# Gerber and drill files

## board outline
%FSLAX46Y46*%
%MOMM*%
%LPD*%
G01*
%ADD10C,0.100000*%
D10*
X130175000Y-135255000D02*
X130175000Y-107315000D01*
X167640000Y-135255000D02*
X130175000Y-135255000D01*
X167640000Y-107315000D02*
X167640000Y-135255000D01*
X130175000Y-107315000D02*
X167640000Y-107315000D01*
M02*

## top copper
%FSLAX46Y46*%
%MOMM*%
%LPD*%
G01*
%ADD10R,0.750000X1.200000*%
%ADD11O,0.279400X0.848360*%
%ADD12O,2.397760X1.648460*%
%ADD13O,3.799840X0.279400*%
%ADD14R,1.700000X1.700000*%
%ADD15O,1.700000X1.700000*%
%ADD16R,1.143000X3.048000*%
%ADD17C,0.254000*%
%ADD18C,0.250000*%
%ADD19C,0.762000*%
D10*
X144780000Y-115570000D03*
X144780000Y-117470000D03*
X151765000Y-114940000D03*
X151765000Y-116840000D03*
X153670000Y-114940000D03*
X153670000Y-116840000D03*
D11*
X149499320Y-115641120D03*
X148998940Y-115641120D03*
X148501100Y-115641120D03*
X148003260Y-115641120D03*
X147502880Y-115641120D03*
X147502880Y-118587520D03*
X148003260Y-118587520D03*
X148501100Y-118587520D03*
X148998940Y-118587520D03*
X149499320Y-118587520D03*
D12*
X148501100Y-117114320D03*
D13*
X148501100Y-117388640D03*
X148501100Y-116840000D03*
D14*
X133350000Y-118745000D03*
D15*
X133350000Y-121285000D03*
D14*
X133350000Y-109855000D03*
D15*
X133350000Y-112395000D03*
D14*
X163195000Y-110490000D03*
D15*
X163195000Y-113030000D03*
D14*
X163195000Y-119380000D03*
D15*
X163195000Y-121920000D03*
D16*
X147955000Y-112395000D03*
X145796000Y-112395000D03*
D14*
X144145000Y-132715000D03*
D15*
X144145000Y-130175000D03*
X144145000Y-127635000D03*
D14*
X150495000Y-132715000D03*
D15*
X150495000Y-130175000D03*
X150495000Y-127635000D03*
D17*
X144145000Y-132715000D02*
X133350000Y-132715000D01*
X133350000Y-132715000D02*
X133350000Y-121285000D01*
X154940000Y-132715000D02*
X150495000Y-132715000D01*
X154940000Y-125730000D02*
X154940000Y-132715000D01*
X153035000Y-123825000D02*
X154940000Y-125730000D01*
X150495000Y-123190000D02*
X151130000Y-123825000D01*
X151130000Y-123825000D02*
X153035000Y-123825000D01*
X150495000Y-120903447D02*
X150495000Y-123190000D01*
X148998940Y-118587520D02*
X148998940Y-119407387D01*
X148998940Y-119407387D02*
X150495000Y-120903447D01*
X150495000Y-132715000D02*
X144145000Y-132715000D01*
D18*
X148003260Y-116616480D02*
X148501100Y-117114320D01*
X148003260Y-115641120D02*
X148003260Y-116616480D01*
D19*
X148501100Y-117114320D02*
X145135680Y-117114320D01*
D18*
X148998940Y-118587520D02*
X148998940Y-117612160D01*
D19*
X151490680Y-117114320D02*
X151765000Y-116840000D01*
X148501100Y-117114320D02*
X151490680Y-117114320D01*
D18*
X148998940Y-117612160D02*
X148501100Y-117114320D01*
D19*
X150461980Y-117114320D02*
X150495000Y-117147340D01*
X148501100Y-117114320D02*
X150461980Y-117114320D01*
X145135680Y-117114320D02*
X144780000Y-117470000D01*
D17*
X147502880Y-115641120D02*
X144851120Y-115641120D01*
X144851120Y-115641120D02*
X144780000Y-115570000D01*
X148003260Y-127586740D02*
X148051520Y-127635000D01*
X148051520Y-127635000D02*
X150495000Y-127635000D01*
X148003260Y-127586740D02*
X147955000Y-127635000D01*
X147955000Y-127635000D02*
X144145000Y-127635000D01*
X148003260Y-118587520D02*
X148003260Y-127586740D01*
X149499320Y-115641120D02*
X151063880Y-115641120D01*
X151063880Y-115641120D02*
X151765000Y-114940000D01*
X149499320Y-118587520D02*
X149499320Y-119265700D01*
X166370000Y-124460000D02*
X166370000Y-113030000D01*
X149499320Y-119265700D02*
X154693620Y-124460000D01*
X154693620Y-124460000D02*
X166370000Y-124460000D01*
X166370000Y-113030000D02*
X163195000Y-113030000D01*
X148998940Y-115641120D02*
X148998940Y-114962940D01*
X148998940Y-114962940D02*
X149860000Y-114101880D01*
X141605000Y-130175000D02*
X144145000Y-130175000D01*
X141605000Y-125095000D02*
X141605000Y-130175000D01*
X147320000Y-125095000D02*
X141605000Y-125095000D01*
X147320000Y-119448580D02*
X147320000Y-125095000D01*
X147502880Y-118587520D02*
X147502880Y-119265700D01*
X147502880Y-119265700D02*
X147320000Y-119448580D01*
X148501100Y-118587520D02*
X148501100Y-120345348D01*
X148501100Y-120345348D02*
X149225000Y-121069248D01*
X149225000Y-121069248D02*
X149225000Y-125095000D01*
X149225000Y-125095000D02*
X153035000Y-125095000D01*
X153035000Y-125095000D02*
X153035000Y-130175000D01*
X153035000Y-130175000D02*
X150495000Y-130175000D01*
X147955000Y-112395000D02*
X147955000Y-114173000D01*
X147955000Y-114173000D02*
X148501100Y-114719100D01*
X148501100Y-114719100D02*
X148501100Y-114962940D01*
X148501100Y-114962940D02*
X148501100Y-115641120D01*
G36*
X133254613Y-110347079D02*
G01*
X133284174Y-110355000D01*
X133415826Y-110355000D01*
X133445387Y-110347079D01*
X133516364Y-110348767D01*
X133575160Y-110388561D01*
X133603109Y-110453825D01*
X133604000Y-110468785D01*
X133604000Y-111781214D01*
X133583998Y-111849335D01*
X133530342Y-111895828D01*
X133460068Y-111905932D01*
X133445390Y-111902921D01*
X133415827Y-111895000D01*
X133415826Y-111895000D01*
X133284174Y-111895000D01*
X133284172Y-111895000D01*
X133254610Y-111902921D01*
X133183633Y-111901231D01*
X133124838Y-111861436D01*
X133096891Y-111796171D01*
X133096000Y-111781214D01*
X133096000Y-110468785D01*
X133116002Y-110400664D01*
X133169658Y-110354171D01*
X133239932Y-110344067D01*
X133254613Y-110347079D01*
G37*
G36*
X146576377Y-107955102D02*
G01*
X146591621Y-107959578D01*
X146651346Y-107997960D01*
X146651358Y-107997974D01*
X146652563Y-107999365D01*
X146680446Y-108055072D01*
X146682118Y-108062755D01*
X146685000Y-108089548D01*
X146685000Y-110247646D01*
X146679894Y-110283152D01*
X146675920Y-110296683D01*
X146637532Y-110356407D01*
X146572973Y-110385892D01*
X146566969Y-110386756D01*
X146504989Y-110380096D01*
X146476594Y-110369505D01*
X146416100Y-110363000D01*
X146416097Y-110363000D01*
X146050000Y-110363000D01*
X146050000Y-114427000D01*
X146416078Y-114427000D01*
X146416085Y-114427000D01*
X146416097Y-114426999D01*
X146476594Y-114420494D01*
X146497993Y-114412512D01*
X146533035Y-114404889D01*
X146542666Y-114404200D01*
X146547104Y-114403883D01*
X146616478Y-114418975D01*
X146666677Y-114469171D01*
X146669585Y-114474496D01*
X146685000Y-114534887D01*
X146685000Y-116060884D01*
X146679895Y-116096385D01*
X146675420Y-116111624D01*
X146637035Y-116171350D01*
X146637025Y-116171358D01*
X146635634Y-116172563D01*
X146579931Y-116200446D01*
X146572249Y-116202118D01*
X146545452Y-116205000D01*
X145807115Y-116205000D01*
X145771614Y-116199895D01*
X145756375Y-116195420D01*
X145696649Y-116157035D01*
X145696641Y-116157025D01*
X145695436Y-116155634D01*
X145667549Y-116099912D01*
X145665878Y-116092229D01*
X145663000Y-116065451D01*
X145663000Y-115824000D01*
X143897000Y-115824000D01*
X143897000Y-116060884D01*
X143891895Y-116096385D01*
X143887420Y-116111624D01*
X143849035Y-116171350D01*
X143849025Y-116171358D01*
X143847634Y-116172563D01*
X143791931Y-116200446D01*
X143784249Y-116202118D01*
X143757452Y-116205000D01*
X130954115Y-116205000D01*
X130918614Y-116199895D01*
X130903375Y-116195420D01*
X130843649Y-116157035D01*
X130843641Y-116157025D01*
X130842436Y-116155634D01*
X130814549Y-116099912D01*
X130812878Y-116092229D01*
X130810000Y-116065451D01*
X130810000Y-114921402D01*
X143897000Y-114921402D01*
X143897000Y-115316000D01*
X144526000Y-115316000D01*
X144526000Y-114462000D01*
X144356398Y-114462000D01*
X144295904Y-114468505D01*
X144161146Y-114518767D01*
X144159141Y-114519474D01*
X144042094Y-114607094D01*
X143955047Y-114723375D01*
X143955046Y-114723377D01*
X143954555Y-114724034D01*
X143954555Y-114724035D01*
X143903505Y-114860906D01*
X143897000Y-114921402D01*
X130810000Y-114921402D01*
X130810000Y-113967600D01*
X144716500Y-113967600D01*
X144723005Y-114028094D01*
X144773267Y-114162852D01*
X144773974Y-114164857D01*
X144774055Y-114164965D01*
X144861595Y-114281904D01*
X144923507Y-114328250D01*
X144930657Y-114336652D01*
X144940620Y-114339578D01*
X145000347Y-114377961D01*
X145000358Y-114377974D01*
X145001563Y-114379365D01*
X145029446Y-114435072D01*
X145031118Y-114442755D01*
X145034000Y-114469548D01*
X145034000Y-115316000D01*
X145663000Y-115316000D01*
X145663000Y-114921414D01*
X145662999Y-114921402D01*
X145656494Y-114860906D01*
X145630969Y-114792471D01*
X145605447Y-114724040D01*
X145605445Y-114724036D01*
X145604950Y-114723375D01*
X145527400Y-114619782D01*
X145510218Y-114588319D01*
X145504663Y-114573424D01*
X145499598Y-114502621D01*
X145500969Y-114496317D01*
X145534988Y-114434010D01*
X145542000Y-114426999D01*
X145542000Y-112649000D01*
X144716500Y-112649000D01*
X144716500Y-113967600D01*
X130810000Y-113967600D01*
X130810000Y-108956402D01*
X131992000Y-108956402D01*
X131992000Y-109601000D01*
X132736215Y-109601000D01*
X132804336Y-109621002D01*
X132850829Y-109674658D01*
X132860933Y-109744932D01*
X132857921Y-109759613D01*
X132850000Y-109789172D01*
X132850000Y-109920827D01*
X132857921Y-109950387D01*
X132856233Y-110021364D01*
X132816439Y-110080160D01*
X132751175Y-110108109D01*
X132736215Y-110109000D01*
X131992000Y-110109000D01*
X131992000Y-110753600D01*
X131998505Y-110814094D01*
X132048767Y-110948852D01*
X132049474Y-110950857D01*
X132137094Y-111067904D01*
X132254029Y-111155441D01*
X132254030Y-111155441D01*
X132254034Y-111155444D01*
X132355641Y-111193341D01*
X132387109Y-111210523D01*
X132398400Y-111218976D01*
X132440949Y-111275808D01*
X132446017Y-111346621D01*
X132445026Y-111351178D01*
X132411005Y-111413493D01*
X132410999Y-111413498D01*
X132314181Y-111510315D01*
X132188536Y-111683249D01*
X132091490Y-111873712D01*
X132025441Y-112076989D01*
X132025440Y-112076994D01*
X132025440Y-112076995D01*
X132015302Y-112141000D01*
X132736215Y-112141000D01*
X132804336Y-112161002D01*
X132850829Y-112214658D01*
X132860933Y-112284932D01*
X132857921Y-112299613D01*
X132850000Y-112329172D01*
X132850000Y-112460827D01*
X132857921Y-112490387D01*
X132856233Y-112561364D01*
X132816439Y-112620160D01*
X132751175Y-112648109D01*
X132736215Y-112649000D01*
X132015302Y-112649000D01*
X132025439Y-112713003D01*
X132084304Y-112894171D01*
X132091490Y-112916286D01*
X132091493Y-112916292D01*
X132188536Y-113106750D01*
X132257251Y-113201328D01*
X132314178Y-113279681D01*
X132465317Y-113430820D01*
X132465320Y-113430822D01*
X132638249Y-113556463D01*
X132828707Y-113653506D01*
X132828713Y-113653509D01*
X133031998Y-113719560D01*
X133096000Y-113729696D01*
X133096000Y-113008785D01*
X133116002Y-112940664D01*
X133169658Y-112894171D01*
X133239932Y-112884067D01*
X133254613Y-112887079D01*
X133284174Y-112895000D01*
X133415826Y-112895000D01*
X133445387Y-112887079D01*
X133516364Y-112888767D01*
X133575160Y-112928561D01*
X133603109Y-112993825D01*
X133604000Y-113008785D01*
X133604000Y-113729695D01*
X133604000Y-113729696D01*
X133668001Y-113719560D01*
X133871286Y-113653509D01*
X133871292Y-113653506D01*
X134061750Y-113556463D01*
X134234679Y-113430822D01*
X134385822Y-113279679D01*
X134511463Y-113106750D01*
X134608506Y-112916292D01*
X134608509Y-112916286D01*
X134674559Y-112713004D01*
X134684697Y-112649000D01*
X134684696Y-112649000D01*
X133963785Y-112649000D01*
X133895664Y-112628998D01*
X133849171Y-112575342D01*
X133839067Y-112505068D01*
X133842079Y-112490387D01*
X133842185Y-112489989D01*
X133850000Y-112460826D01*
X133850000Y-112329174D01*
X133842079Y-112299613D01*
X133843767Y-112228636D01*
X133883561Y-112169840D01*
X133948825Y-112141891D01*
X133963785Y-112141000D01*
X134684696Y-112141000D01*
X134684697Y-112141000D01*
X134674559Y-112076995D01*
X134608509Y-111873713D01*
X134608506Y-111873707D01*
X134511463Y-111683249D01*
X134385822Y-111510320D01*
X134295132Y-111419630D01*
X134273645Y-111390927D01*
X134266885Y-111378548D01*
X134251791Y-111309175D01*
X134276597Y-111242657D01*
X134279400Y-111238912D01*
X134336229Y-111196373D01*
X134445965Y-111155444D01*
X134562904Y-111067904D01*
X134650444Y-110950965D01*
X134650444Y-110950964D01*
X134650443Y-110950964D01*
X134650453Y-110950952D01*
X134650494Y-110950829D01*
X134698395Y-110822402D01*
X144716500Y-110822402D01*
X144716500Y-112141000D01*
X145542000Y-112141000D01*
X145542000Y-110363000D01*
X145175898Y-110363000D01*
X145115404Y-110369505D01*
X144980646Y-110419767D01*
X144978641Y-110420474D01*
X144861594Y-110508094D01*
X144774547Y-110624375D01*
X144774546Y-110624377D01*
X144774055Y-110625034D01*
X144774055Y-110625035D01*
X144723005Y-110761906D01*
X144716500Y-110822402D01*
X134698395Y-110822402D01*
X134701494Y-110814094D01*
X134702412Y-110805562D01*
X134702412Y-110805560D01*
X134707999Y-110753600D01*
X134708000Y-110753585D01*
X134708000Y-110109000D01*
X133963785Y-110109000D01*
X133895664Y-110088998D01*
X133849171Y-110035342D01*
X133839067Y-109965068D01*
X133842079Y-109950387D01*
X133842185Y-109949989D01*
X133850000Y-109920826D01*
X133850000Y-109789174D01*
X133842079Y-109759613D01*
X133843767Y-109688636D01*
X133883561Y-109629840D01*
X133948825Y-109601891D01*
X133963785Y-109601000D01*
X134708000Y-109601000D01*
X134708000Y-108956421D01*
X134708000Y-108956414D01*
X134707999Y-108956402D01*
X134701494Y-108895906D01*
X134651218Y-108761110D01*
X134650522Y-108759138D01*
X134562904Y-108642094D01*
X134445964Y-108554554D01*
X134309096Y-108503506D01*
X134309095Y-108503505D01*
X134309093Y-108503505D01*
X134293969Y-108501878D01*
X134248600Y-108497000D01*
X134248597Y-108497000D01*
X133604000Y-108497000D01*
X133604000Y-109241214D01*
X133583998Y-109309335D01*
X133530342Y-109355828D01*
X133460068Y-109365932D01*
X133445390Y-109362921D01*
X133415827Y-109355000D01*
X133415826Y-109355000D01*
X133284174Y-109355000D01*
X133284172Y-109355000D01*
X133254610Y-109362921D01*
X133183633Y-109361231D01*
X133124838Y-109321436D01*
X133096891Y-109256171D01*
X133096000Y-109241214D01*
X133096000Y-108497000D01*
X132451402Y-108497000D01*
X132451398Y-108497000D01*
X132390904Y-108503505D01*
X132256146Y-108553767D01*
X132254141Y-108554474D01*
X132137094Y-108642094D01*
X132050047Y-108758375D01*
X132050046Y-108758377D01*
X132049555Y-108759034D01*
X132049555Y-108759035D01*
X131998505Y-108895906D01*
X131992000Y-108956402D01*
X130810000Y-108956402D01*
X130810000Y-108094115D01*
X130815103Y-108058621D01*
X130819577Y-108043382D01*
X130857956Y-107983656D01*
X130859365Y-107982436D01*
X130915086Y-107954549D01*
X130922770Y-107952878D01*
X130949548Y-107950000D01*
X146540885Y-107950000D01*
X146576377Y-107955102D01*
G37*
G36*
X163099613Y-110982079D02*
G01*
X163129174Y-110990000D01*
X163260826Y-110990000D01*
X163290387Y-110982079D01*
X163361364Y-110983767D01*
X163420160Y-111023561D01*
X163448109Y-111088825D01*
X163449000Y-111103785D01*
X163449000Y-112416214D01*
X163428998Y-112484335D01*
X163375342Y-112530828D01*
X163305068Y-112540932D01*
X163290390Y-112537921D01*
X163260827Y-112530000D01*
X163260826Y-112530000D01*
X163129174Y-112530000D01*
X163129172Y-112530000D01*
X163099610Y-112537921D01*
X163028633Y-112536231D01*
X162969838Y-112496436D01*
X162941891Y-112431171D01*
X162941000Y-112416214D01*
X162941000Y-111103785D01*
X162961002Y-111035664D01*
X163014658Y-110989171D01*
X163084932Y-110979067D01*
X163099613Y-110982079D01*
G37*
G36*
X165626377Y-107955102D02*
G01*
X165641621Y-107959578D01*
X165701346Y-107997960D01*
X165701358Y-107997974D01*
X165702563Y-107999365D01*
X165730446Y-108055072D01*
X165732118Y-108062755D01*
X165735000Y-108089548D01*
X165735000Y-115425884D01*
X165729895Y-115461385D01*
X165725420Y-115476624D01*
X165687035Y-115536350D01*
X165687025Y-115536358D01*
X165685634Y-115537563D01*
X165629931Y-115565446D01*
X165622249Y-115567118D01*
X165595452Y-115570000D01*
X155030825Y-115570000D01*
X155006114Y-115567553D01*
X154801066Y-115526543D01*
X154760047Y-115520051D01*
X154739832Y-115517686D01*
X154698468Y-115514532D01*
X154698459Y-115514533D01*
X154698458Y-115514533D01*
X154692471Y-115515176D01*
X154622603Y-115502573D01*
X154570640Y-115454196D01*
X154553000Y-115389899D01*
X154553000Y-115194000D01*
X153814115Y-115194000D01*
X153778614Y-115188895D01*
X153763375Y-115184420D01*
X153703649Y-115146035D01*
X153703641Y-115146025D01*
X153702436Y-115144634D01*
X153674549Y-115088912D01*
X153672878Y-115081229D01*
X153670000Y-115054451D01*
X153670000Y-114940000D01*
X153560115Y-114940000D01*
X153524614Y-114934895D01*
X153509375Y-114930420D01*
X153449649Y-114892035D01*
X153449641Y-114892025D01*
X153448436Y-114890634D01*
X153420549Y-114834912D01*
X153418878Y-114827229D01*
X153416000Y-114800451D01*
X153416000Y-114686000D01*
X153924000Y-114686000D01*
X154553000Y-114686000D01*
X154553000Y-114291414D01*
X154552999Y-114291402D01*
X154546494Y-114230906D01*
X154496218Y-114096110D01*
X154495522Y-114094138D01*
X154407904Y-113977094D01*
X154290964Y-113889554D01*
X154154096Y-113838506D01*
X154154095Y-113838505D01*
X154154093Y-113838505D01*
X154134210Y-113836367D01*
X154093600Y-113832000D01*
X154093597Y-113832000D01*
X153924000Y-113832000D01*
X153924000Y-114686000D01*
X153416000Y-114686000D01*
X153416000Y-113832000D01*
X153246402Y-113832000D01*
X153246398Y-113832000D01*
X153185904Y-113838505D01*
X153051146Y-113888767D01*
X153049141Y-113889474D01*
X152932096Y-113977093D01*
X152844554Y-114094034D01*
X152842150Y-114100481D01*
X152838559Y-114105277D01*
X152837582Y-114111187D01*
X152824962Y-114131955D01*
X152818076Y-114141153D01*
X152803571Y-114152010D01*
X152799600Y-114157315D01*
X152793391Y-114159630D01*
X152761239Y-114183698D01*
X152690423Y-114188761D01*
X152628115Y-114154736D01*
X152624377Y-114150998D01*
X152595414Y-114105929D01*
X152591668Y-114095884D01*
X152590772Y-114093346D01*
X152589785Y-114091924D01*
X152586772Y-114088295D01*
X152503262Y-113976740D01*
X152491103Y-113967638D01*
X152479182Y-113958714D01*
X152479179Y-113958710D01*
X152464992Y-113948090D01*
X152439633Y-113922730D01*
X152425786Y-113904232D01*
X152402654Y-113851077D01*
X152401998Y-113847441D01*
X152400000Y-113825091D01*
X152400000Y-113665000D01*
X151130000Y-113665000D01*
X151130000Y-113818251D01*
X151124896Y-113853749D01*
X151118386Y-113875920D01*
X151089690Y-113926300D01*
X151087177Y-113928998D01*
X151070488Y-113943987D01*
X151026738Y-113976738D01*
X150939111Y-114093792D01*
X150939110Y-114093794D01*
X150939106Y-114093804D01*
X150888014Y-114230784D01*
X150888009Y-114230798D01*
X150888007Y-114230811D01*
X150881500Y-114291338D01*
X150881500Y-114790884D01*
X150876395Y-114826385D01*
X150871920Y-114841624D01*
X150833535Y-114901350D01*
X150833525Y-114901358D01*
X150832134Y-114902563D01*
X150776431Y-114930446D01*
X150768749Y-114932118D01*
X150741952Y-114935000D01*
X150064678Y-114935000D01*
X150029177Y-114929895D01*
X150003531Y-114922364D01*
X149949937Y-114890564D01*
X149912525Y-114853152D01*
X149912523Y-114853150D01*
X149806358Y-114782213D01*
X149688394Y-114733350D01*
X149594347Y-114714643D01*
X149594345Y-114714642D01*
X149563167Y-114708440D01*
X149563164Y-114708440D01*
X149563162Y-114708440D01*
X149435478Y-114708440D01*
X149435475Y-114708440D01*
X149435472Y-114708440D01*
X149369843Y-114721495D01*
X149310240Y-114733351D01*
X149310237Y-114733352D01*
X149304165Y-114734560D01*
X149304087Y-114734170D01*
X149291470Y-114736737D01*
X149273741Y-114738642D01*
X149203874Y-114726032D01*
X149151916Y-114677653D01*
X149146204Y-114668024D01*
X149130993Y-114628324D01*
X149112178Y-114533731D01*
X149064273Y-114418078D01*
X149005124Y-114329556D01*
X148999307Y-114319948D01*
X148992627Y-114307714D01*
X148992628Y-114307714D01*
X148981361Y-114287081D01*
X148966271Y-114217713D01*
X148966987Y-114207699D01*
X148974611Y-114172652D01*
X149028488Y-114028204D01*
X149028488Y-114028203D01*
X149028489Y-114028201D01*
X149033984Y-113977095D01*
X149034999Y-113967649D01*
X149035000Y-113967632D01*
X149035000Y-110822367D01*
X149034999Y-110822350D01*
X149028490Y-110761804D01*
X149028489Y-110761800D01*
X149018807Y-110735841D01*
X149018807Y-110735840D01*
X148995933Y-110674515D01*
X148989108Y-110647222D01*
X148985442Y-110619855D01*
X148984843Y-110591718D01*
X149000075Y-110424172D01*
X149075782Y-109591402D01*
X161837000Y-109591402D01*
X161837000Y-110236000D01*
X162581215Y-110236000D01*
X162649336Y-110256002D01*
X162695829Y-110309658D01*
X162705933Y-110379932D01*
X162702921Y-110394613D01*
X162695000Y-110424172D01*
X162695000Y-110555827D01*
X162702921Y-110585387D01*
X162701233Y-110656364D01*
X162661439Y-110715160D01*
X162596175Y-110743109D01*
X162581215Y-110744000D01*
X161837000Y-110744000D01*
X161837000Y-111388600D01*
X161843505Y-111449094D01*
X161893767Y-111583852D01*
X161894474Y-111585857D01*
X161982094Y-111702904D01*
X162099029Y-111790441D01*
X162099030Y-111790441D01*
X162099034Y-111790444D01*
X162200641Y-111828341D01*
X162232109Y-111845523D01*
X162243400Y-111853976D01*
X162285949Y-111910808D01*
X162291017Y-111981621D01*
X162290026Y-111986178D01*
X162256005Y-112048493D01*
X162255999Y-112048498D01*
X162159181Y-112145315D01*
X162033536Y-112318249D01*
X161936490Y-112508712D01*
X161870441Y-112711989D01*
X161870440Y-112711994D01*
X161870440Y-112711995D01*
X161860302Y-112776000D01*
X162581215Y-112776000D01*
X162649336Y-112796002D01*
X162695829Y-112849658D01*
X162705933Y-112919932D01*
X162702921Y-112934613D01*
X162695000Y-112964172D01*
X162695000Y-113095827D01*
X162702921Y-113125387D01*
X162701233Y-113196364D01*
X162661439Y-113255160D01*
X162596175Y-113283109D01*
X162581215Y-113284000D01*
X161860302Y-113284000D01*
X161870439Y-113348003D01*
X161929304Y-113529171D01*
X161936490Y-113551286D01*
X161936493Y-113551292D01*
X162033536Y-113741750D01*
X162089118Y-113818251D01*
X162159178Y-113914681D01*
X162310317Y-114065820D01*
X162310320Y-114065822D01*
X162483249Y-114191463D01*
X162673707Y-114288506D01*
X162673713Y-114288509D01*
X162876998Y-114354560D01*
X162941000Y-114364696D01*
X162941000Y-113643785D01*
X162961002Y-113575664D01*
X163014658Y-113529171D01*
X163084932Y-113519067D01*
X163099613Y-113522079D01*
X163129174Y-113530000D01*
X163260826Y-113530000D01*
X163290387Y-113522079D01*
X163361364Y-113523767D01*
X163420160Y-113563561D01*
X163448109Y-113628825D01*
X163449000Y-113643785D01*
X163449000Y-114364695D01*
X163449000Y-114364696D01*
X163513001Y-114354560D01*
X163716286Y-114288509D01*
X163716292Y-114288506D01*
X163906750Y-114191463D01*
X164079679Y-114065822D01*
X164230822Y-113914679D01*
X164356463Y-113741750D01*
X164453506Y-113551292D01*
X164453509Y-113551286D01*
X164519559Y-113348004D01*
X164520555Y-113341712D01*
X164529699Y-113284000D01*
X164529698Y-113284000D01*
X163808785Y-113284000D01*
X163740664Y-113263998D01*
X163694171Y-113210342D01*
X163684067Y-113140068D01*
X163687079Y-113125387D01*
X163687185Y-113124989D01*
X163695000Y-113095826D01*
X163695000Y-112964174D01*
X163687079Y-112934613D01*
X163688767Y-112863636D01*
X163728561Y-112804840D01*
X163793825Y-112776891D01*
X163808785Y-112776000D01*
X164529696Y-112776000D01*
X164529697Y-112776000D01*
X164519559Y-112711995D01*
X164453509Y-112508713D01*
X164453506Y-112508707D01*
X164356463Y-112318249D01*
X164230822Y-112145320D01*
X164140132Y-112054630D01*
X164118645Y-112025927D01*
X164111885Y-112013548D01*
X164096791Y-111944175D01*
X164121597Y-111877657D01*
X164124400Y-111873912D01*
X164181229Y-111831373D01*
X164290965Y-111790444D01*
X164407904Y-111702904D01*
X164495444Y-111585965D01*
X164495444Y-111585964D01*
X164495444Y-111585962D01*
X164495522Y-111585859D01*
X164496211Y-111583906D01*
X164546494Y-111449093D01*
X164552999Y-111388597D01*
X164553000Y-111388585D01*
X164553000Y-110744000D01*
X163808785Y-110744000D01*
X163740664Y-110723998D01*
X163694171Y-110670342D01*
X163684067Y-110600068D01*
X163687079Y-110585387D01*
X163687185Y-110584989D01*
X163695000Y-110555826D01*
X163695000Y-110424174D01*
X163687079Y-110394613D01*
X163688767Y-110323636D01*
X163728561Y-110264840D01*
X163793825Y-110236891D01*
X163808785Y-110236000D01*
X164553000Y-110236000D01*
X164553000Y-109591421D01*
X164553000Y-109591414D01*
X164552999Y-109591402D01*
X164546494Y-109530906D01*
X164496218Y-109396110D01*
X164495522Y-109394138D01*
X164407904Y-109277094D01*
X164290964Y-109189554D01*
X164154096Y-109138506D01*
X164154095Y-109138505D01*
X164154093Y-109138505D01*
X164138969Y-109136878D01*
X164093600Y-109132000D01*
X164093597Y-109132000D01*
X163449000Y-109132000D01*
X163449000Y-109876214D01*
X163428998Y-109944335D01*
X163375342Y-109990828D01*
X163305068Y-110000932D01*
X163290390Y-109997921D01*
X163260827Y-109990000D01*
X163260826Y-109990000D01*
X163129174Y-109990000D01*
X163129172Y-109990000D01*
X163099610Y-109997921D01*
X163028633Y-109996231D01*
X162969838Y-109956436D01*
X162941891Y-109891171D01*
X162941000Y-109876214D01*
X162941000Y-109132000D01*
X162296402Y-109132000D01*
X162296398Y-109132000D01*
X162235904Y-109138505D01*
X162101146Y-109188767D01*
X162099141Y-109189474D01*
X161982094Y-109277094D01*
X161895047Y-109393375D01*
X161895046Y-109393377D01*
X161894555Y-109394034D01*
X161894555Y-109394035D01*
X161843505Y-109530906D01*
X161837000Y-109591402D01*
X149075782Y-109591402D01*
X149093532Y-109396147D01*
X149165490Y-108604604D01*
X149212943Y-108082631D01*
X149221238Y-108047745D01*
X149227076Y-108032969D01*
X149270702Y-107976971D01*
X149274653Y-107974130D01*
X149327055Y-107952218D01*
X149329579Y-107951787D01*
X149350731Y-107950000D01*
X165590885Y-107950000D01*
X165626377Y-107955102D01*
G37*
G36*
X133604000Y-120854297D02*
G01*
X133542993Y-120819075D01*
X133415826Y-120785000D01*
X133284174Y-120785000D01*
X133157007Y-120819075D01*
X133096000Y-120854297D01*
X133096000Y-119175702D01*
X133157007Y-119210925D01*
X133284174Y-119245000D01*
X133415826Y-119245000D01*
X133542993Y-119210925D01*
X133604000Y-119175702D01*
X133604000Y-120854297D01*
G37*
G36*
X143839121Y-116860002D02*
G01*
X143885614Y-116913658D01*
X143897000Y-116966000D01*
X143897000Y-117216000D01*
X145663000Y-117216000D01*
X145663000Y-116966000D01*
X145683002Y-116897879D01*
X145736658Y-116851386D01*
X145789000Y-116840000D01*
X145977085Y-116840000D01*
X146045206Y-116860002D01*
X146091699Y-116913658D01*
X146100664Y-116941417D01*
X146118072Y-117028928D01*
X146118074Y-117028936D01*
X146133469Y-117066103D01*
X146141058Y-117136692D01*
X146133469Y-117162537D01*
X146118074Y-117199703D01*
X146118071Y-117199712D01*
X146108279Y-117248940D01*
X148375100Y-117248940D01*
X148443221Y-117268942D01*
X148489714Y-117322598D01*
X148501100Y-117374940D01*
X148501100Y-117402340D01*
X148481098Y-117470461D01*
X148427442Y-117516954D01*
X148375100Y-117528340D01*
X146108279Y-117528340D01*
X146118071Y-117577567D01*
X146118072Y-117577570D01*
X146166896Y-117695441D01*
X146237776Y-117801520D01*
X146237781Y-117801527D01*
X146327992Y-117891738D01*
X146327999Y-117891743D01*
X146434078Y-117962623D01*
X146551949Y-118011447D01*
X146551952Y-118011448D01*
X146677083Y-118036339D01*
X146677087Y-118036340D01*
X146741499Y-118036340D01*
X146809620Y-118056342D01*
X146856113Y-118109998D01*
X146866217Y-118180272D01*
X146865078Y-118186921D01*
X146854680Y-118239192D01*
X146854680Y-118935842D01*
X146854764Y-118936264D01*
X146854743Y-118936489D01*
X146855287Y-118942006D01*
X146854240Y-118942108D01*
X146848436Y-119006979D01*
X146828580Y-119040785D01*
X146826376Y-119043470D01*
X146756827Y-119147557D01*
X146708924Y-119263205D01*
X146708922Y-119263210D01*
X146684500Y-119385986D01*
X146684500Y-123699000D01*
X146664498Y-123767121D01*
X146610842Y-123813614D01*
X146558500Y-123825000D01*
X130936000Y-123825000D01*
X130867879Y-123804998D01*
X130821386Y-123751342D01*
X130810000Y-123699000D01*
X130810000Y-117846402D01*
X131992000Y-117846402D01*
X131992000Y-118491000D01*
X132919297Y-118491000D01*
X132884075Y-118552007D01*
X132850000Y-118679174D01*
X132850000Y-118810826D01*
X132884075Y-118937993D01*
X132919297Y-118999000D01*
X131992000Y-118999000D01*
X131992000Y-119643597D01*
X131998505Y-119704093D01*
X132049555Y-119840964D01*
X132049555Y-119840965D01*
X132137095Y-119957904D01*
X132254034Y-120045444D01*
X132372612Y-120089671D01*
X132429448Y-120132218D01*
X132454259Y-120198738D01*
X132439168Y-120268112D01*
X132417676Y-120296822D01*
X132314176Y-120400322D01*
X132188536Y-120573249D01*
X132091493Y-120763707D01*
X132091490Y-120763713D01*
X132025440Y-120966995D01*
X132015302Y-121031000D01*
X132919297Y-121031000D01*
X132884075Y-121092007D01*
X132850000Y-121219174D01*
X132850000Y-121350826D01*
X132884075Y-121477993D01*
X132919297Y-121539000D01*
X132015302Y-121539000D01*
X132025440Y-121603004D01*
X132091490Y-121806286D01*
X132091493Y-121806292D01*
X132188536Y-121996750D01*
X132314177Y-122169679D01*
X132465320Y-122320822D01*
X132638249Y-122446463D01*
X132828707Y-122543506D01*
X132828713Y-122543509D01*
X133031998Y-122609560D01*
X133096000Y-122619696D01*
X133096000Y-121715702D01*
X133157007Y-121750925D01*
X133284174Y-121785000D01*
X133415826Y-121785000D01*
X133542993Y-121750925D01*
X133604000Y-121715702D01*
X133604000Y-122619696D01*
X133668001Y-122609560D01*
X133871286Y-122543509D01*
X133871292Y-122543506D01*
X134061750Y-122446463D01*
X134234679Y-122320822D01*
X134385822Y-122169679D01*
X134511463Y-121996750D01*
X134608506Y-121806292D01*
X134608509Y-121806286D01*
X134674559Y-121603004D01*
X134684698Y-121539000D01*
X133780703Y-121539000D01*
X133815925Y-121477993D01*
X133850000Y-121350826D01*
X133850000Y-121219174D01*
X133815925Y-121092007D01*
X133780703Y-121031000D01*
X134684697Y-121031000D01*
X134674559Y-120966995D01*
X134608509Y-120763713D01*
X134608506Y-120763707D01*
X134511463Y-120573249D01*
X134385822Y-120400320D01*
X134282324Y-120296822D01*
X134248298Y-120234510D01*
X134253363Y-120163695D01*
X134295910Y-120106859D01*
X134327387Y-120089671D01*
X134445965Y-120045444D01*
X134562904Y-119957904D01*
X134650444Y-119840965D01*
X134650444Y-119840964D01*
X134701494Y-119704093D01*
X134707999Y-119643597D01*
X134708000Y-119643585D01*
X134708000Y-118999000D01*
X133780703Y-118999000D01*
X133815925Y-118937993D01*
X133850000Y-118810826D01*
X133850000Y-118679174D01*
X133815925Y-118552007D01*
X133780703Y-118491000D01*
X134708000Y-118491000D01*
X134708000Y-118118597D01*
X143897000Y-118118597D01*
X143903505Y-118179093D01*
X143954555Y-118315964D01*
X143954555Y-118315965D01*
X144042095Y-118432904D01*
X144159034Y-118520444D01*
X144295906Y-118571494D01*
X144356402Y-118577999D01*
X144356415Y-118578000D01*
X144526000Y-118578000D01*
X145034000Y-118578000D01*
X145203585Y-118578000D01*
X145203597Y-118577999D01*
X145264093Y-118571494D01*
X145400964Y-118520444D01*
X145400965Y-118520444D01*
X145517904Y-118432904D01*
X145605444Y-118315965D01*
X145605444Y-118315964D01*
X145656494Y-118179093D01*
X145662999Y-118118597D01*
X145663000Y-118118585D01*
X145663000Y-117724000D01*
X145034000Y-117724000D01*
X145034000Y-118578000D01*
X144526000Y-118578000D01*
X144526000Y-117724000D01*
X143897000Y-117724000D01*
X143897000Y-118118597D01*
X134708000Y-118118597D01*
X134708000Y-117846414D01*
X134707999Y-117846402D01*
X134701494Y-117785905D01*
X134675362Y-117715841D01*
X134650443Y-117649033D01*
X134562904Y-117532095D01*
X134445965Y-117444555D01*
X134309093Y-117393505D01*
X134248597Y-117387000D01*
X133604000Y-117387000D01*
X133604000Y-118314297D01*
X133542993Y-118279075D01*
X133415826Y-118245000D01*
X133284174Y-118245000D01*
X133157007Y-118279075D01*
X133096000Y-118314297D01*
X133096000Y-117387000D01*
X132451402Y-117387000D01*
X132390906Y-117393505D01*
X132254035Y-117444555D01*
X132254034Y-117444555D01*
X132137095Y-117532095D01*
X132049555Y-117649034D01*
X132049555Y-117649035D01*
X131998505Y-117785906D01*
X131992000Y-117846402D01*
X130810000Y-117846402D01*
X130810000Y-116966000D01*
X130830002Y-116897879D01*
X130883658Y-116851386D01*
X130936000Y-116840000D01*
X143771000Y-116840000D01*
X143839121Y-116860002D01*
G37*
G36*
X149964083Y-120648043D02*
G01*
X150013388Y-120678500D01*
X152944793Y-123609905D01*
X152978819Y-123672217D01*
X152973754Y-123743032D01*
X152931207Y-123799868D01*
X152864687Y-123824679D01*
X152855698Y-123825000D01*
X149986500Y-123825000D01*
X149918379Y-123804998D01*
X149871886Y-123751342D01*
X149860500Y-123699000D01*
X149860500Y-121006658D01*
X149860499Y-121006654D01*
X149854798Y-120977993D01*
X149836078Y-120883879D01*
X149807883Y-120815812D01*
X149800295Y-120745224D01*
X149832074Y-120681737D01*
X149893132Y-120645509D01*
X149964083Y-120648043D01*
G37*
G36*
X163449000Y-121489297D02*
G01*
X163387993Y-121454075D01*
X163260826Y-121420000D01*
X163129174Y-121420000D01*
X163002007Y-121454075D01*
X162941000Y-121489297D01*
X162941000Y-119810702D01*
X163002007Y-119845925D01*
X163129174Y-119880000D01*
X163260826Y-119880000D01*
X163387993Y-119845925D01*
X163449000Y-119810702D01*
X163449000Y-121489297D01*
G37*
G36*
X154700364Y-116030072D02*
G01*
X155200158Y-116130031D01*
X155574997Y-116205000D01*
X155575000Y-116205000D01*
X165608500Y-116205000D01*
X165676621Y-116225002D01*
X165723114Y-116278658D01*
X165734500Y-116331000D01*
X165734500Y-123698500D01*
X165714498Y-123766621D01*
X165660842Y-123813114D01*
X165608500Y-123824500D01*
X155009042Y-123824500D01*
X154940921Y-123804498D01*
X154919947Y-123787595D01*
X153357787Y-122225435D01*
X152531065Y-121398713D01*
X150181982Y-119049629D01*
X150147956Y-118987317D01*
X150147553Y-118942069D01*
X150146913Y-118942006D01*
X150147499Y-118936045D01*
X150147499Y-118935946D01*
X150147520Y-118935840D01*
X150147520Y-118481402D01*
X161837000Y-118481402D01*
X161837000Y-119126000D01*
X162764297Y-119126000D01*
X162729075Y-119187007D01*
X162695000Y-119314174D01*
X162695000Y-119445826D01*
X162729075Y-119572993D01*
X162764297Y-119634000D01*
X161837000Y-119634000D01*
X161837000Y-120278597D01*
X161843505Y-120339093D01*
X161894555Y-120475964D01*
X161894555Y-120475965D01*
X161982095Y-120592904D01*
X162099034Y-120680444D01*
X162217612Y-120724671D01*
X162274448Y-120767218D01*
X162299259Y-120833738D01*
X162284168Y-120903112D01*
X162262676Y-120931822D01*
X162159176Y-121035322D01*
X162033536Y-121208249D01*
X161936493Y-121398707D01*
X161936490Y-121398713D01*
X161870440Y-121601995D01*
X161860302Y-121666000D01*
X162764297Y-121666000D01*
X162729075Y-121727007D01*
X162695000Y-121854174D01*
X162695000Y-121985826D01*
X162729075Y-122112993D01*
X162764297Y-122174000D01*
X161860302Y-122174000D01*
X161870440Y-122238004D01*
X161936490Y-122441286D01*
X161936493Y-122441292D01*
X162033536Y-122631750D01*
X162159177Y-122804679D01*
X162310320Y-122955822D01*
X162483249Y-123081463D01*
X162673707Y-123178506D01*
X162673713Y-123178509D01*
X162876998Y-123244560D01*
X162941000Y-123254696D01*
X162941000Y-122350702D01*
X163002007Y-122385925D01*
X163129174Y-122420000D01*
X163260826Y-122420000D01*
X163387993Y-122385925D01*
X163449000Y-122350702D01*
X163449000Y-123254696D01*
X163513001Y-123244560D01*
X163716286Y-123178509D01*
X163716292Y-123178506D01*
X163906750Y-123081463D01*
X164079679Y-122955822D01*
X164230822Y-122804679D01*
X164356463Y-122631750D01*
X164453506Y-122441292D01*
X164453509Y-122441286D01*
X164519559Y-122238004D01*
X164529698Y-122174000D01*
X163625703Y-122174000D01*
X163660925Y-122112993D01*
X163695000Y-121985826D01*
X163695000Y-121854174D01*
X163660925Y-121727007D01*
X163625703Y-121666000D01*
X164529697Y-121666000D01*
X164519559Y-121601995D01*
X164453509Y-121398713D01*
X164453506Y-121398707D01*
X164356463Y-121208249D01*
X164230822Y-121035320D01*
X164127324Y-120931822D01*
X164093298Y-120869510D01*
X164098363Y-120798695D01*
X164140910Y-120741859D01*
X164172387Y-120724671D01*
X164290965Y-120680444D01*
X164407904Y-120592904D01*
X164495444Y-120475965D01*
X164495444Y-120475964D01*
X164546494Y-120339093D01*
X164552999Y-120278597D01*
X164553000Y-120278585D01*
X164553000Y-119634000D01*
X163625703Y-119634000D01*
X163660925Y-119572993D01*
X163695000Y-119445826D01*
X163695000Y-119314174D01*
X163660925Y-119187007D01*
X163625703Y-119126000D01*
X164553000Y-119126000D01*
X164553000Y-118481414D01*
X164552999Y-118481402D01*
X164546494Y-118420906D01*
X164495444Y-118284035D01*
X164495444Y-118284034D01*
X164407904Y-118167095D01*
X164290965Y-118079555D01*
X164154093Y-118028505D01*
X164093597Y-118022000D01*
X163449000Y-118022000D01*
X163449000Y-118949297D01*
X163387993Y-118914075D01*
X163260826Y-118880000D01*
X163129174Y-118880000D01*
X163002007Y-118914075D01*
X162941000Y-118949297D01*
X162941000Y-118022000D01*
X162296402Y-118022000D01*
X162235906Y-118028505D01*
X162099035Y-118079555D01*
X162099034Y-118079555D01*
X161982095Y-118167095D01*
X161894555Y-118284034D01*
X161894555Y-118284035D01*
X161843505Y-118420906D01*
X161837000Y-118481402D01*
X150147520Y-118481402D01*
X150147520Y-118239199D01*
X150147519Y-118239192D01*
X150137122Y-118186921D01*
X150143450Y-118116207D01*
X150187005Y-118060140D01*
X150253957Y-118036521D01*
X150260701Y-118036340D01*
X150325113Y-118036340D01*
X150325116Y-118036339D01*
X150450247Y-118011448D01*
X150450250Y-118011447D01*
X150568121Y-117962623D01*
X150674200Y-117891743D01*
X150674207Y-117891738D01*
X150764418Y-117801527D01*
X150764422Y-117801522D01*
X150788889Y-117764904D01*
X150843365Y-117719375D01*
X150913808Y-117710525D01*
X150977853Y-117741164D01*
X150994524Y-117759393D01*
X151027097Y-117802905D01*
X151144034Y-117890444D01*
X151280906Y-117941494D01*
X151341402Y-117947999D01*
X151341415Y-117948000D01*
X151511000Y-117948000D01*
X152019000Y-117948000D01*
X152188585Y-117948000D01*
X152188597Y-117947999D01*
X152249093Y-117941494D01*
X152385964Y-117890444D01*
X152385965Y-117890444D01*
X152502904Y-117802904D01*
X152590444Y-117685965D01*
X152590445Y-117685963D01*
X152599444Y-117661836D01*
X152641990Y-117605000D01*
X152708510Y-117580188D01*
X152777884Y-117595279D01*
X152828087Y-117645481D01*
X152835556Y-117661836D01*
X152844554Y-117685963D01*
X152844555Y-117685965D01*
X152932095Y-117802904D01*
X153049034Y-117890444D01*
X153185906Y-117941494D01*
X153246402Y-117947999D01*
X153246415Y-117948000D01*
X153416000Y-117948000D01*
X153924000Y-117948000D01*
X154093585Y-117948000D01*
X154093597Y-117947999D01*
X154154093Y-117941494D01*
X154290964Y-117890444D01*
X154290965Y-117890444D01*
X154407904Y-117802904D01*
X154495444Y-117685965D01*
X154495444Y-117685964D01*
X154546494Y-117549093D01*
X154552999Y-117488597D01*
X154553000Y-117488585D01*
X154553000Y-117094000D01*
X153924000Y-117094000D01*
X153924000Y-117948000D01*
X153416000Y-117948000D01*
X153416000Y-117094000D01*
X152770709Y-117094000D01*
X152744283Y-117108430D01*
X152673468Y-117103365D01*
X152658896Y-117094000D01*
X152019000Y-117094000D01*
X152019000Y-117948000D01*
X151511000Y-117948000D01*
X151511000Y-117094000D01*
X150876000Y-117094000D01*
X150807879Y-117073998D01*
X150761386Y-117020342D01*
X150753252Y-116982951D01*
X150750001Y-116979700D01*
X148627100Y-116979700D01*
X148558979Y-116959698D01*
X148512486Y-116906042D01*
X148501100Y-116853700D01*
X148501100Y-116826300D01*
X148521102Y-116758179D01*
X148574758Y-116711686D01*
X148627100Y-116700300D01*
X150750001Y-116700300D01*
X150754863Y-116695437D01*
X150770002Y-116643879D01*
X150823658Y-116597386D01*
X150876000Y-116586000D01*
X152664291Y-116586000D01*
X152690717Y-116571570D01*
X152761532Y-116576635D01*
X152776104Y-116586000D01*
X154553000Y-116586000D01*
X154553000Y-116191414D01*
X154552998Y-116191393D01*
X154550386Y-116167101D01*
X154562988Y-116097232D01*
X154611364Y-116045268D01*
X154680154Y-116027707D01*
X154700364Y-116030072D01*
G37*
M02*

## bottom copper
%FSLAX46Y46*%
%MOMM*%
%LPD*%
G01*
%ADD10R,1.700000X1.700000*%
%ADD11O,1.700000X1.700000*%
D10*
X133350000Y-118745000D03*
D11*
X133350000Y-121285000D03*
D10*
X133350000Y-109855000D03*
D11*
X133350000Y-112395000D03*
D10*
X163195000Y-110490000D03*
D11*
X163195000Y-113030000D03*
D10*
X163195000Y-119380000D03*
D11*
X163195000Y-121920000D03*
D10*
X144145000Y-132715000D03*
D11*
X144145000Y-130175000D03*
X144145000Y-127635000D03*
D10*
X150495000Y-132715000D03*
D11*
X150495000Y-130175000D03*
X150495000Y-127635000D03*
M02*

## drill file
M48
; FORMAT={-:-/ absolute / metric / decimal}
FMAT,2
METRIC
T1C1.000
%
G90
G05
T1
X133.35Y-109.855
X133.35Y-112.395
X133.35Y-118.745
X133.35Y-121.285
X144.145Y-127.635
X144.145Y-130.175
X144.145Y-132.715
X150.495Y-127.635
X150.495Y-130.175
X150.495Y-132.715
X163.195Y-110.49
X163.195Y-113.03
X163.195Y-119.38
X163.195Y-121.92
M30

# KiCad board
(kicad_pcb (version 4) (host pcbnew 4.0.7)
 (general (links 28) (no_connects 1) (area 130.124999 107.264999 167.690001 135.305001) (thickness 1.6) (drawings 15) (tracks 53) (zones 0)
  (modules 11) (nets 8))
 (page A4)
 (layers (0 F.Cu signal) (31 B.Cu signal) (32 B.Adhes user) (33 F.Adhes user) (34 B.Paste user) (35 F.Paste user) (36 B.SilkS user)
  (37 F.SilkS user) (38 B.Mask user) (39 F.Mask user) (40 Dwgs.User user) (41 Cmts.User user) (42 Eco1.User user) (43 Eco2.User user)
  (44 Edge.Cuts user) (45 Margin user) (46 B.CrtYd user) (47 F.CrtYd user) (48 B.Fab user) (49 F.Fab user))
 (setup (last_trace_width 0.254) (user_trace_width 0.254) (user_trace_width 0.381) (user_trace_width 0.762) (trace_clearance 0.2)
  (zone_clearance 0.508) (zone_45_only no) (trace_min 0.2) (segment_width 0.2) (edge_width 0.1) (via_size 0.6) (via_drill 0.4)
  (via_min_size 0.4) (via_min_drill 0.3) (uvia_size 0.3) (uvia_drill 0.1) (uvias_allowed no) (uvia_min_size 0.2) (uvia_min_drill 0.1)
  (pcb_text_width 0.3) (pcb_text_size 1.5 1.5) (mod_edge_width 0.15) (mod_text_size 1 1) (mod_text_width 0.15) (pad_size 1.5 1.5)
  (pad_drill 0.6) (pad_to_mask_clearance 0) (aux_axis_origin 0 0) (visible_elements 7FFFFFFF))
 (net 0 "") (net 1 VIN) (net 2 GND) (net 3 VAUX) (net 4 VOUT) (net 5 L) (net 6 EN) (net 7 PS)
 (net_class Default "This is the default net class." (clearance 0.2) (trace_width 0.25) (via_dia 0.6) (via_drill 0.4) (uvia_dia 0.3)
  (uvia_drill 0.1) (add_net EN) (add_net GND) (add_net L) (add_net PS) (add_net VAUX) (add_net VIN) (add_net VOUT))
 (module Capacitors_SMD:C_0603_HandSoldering (layer F.Cu) (at 144.78 116.52 270)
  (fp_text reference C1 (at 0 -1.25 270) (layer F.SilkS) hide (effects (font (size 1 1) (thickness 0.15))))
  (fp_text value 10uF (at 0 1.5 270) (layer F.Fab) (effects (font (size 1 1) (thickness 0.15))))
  (pad 1 smd rect (at -0.95 0 270) (size 1.2 0.75) (layers F.Cu F.Paste F.Mask) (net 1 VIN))
  (pad 2 smd rect (at 0.95 0 270) (size 1.2 0.75) (layers F.Cu F.Paste F.Mask) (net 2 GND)))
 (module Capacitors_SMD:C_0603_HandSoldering (layer F.Cu) (at 151.765 115.89 270)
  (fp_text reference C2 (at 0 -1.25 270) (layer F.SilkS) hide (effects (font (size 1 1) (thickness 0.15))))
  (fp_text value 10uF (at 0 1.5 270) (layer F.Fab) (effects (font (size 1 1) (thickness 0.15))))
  (pad 1 smd rect (at -0.95 0 270) (size 1.2 0.75) (layers F.Cu F.Paste F.Mask) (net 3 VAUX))
  (pad 2 smd rect (at 0.95 0 270) (size 1.2 0.75) (layers F.Cu F.Paste F.Mask) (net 2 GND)))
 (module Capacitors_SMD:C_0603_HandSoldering (layer F.Cu) (at 153.67 115.89 270)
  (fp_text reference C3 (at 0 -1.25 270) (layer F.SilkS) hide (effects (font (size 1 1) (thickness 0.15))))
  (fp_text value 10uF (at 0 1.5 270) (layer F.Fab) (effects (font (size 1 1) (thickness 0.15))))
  (pad 1 smd rect (at -0.95 0 270) (size 1.2 0.75) (layers F.Cu F.Paste F.Mask) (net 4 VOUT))
  (pad 2 smd rect (at 0.95 0 270) (size 1.2 0.75) (layers F.Cu F.Paste F.Mask) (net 2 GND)))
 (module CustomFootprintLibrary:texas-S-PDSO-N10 (layer F.Cu) (at 148.5011 117.11432 180)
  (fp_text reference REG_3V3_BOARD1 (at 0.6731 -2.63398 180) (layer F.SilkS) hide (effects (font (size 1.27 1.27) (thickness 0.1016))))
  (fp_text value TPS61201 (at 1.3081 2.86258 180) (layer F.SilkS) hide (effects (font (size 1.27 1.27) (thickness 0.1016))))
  (pad 1 smd oval (at -0.99822 1.4732 270) (size 0.84836 0.2794) (layers F.Cu F.Paste F.Mask) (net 3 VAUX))
  (pad 2 smd oval (at -0.49784 1.4732 270) (size 0.84836 0.2794) (layers F.Cu F.Paste F.Mask) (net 4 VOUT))
  (pad 3 smd oval (at 0 1.4732 270) (size 0.84836 0.2794) (layers F.Cu F.Paste F.Mask) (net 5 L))
  (pad 4 smd oval (at 0.49784 1.4732 270) (size 0.84836 0.2794) (layers F.Cu F.Paste F.Mask) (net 2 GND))
  (pad 5 smd oval (at 0.99822 1.4732 270) (size 0.84836 0.2794) (layers F.Cu F.Paste F.Mask) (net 1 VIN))
  (pad 6 smd oval (at 0.99822 -1.4732 90) (size 0.84836 0.2794) (layers F.Cu F.Paste F.Mask) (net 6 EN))
  (pad 7 smd oval (at 0.49784 -1.4732 90) (size 0.84836 0.2794) (layers F.Cu F.Paste F.Mask) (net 1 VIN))
  (pad 8 smd oval (at 0 -1.4732 90) (size 0.84836 0.2794) (layers F.Cu F.Paste F.Mask) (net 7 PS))
  (pad 9 smd oval (at -0.49784 -1.4732 90) (size 0.84836 0.2794) (layers F.Cu F.Paste F.Mask) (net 2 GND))
  (pad 10 smd oval (at -0.99822 -1.4732 90) (size 0.84836 0.2794) (layers F.Cu F.Paste F.Mask) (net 4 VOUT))
  (pad PP smd oval (at 0 0 180) (size 2.39776 1.64846) (layers F.Cu F.Paste F.Mask) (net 2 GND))
  (pad PP@1 smd oval (at 0 -0.27432 180) (size 3.79984 0.2794) (layers F.Cu F.Paste F.Mask) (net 2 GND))
  (pad PP@2 smd oval (at 0 0.27432 180) (size 3.79984 0.2794) (layers F.Cu F.Paste F.Mask) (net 2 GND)))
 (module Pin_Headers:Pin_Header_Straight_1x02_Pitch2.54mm (layer F.Cu) (at 133.35 118.745)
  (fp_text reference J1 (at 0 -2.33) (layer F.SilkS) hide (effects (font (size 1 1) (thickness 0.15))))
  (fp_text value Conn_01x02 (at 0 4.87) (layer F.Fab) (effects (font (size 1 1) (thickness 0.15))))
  (pad 1 thru_hole rect (at 0 0) (size 1.7 1.7) (drill 1) (layers *.Cu *.Mask) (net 2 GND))
  (pad 2 thru_hole oval (at 0 2.54) (size 1.7 1.7) (drill 1) (layers *.Cu *.Mask) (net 2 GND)))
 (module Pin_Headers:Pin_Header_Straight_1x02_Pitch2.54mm (layer F.Cu) (at 133.35 109.855)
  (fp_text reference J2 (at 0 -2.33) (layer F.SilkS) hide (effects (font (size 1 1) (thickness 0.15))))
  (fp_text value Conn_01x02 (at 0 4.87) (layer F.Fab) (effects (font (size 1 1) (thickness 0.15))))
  (pad 1 thru_hole rect (at 0 0) (size 1.7 1.7) (drill 1) (layers *.Cu *.Mask) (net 1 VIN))
  (pad 2 thru_hole oval (at 0 2.54) (size 1.7 1.7) (drill 1) (layers *.Cu *.Mask) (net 1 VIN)))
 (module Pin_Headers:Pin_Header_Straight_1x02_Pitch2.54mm (layer F.Cu) (at 163.195 110.49)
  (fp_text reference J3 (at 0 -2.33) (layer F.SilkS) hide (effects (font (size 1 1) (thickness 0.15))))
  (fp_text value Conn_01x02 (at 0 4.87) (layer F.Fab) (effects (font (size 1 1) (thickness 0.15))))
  (pad 1 thru_hole rect (at 0 0) (size 1.7 1.7) (drill 1) (layers *.Cu *.Mask) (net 4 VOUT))
  (pad 2 thru_hole oval (at 0 2.54) (size 1.7 1.7) (drill 1) (layers *.Cu *.Mask) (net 4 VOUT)))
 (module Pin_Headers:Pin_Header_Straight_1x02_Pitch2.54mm (layer F.Cu) (at 163.195 119.38)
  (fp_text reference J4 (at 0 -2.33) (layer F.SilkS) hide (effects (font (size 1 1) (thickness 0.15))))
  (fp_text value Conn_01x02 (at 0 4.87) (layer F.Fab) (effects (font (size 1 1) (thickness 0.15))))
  (pad 1 thru_hole rect (at 0 0) (size 1.7 1.7) (drill 1) (layers *.Cu *.Mask) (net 2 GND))
  (pad 2 thru_hole oval (at 0 2.54) (size 1.7 1.7) (drill 1) (layers *.Cu *.Mask) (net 2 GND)))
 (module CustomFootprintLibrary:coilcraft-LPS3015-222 (layer F.Cu) (at 146.8755 112.395)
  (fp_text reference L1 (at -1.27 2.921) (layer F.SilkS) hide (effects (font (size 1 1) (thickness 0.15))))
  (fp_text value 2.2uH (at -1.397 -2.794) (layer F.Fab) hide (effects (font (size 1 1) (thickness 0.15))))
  (pad 2 smd rect (at 1.0795 0) (size 1.143 3.048) (layers F.Cu F.Paste F.Mask) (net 5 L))
  (pad 1 smd rect (at -1.0795 0) (size 1.143 3.048) (layers F.Cu F.Paste F.Mask) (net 1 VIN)))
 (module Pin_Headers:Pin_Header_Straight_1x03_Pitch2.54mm (layer F.Cu) (at 144.145 132.715 180)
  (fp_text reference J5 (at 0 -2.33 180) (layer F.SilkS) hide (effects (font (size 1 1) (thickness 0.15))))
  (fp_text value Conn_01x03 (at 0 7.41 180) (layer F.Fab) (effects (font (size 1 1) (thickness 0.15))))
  (pad 1 thru_hole rect (at 0 0 180) (size 1.7 1.7) (drill 1) (layers *.Cu *.Mask) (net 2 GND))
  (pad 2 thru_hole oval (at 0 2.54 180) (size 1.7 1.7) (drill 1) (layers *.Cu *.Mask) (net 6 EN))
  (pad 3 thru_hole oval (at 0 5.08 180) (size 1.7 1.7) (drill 1) (layers *.Cu *.Mask) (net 1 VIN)))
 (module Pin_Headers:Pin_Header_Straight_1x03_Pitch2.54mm (layer F.Cu) (at 150.495 132.715 180)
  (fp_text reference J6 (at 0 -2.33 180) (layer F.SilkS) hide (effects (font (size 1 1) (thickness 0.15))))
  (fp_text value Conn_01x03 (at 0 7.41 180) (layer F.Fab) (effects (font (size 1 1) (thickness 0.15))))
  (pad 1 thru_hole rect (at 0 0 180) (size 1.7 1.7) (drill 1) (layers *.Cu *.Mask) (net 2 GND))
  (pad 2 thru_hole oval (at 0 2.54 180) (size 1.7 1.7) (drill 1) (layers *.Cu *.Mask) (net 7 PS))
  (pad 3 thru_hole oval (at 0 5.08 180) (size 1.7 1.7) (drill 1) (layers *.Cu *.Mask) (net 1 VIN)))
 (gr_line (start 130.175 135.255) (end 130.175 107.315) (angle 90) (layer Edge.Cuts) (width 0.1))
 (gr_line (start 167.64 135.255) (end 130.175 135.255) (angle 90) (layer Edge.Cuts) (width 0.1))
 (gr_line (start 167.64 107.315) (end 167.64 135.255) (angle 90) (layer Edge.Cuts) (width 0.1))
 (gr_line (start 130.175 107.315) (end 167.64 107.315) (angle 90) (layer Edge.Cuts) (width 0.1))
 (segment (start 144.145 132.715) (end 133.35 132.715) (width 0.254) (layer F.Cu) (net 2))
 (segment (start 133.35 132.715) (end 133.35 121.285) (width 0.254) (layer F.Cu) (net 2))
 (segment (start 154.94 132.715) (end 150.495 132.715) (width 0.254) (layer F.Cu) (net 2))
 (segment (start 154.94 125.73) (end 154.94 132.715) (width 0.254) (layer F.Cu) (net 2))
 (segment (start 153.035 123.825) (end 154.94 125.73) (width 0.254) (layer F.Cu) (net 2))
 (segment (start 150.495 123.19) (end 151.13 123.825) (width 0.254) (layer F.Cu) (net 2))
 (segment (start 151.13 123.825) (end 153.035 123.825) (width 0.254) (layer F.Cu) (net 2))
 (segment (start 150.495 120.903447) (end 150.495 123.19) (width 0.254) (layer F.Cu) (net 2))
 (segment (start 148.99894 118.58752) (end 148.99894 119.407387) (width 0.254) (layer F.Cu) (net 2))
 (segment (start 148.99894 119.407387) (end 150.495 120.903447) (width 0.254) (layer F.Cu) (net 2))
 (segment (start 150.495 132.715) (end 144.145 132.715) (width 0.254) (layer F.Cu) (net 2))
 (segment (start 148.00326 116.61648) (end 148.5011 117.11432) (width 0.25) (layer F.Cu) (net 2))
 (segment (start 148.00326 115.64112) (end 148.00326 116.61648) (width 0.25) (layer F.Cu) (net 2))
 (segment (start 148.5011 117.11432) (end 145.13568 117.11432) (width 0.762) (layer F.Cu) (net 2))
 (segment (start 148.99894 118.58752) (end 148.99894 117.61216) (width 0.25) (layer F.Cu) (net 2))
 (segment (start 151.49068 117.11432) (end 151.765 116.84) (width 0.762) (layer F.Cu) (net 2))
 (segment (start 148.5011 117.11432) (end 151.49068 117.11432) (width 0.762) (layer F.Cu) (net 2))
 (segment (start 148.99894 117.61216) (end 148.5011 117.11432) (width 0.25) (layer F.Cu) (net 2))
 (segment (start 150.46198 117.11432) (end 150.495 117.14734) (width 0.762) (layer F.Cu) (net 2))
 (segment (start 148.5011 117.11432) (end 150.46198 117.11432) (width 0.762) (layer F.Cu) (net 2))
 (segment (start 145.13568 117.11432) (end 144.78 117.47) (width 0.762) (layer F.Cu) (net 2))
 (segment (start 147.50288 115.64112) (end 144.85112 115.64112) (width 0.254) (layer F.Cu) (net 1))
 (segment (start 144.85112 115.64112) (end 144.78 115.57) (width 0.254) (layer F.Cu) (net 1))
 (segment (start 148.00326 127.58674) (end 148.05152 127.635) (width 0.254) (layer F.Cu) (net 1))
 (segment (start 148.05152 127.635) (end 150.495 127.635) (width 0.254) (layer F.Cu) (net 1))
 (segment (start 148.00326 127.58674) (end 147.955 127.635) (width 0.254) (layer F.Cu) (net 1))
 (segment (start 147.955 127.635) (end 144.145 127.635) (width 0.254) (layer F.Cu) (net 1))
 (segment (start 148.00326 118.58752) (end 148.00326 127.58674) (width 0.254) (layer F.Cu) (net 1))
 (segment (start 149.49932 115.64112) (end 151.06388 115.64112) (width 0.254) (layer F.Cu) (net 3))
 (segment (start 151.06388 115.64112) (end 151.765 114.94) (width 0.254) (layer F.Cu) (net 3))
 (segment (start 149.49932 118.58752) (end 149.49932 119.2657) (width 0.254) (layer F.Cu) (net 4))
 (segment (start 166.37 124.46) (end 166.37 113.03) (width 0.254) (layer F.Cu) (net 4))
 (segment (start 149.49932 119.2657) (end 154.69362 124.46) (width 0.254) (layer F.Cu) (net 4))
 (segment (start 154.69362 124.46) (end 166.37 124.46) (width 0.254) (layer F.Cu) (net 4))
 (segment (start 166.37 113.03) (end 163.195 113.03) (width 0.254) (layer F.Cu) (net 4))
 (segment (start 148.99894 115.64112) (end 148.99894 114.96294) (width 0.254) (layer F.Cu) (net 4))
 (segment (start 148.99894 114.96294) (end 149.86 114.10188) (width 0.254) (layer F.Cu) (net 4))
 (segment (start 141.605 130.175) (end 144.145 130.175) (width 0.254) (layer F.Cu) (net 6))
 (segment (start 141.605 125.095) (end 141.605 130.175) (width 0.254) (layer F.Cu) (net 6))
 (segment (start 147.32 125.095) (end 141.605 125.095) (width 0.254) (layer F.Cu) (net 6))
 (segment (start 147.32 119.44858) (end 147.32 125.095) (width 0.254) (layer F.Cu) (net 6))
 (segment (start 147.50288 118.58752) (end 147.50288 119.2657) (width 0.254) (layer F.Cu) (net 6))
 (segment (start 147.50288 119.2657) (end 147.32 119.44858) (width 0.254) (layer F.Cu) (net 6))
 (segment (start 148.5011 118.58752) (end 148.5011 120.345348) (width 0.254) (layer F.Cu) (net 7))
 (segment (start 148.5011 120.345348) (end 149.225 121.069248) (width 0.254) (layer F.Cu) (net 7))
 (segment (start 149.225 121.069248) (end 149.225 125.095) (width 0.254) (layer F.Cu) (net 7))
 (segment (start 149.225 125.095) (end 153.035 125.095) (width 0.254) (layer F.Cu) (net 7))
 (segment (start 153.035 125.095) (end 153.035 130.175) (width 0.254) (layer F.Cu) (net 7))
 (segment (start 153.035 130.175) (end 150.495 130.175) (width 0.254) (layer F.Cu) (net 7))
 (segment (start 147.955 112.395) (end 147.955 114.173) (width 0.254) (layer F.Cu) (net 5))
 (segment (start 147.955 114.173) (end 148.5011 114.7191) (width 0.254) (layer F.Cu) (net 5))
 (segment (start 148.5011 114.7191) (end 148.5011 114.96294) (width 0.254) (layer F.Cu) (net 5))
 (segment (start 148.5011 114.96294) (end 148.5011 115.64112) (width 0.254) (layer F.Cu) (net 5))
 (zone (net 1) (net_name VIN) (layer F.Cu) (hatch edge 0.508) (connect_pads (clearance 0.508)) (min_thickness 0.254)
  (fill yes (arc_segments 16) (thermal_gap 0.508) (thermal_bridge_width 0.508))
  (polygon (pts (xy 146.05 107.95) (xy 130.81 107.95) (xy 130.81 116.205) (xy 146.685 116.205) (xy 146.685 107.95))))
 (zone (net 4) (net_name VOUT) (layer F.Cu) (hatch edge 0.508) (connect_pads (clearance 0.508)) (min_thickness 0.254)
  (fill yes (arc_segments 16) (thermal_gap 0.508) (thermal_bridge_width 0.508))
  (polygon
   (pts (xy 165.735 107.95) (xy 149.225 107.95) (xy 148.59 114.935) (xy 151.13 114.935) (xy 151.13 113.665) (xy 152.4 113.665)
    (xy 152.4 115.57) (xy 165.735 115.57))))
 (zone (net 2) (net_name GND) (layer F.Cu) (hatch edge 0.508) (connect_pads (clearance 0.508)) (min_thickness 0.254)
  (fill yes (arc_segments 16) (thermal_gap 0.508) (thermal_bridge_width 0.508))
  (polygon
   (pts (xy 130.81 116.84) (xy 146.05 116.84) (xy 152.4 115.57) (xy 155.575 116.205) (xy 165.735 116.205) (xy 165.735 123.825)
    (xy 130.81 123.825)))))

